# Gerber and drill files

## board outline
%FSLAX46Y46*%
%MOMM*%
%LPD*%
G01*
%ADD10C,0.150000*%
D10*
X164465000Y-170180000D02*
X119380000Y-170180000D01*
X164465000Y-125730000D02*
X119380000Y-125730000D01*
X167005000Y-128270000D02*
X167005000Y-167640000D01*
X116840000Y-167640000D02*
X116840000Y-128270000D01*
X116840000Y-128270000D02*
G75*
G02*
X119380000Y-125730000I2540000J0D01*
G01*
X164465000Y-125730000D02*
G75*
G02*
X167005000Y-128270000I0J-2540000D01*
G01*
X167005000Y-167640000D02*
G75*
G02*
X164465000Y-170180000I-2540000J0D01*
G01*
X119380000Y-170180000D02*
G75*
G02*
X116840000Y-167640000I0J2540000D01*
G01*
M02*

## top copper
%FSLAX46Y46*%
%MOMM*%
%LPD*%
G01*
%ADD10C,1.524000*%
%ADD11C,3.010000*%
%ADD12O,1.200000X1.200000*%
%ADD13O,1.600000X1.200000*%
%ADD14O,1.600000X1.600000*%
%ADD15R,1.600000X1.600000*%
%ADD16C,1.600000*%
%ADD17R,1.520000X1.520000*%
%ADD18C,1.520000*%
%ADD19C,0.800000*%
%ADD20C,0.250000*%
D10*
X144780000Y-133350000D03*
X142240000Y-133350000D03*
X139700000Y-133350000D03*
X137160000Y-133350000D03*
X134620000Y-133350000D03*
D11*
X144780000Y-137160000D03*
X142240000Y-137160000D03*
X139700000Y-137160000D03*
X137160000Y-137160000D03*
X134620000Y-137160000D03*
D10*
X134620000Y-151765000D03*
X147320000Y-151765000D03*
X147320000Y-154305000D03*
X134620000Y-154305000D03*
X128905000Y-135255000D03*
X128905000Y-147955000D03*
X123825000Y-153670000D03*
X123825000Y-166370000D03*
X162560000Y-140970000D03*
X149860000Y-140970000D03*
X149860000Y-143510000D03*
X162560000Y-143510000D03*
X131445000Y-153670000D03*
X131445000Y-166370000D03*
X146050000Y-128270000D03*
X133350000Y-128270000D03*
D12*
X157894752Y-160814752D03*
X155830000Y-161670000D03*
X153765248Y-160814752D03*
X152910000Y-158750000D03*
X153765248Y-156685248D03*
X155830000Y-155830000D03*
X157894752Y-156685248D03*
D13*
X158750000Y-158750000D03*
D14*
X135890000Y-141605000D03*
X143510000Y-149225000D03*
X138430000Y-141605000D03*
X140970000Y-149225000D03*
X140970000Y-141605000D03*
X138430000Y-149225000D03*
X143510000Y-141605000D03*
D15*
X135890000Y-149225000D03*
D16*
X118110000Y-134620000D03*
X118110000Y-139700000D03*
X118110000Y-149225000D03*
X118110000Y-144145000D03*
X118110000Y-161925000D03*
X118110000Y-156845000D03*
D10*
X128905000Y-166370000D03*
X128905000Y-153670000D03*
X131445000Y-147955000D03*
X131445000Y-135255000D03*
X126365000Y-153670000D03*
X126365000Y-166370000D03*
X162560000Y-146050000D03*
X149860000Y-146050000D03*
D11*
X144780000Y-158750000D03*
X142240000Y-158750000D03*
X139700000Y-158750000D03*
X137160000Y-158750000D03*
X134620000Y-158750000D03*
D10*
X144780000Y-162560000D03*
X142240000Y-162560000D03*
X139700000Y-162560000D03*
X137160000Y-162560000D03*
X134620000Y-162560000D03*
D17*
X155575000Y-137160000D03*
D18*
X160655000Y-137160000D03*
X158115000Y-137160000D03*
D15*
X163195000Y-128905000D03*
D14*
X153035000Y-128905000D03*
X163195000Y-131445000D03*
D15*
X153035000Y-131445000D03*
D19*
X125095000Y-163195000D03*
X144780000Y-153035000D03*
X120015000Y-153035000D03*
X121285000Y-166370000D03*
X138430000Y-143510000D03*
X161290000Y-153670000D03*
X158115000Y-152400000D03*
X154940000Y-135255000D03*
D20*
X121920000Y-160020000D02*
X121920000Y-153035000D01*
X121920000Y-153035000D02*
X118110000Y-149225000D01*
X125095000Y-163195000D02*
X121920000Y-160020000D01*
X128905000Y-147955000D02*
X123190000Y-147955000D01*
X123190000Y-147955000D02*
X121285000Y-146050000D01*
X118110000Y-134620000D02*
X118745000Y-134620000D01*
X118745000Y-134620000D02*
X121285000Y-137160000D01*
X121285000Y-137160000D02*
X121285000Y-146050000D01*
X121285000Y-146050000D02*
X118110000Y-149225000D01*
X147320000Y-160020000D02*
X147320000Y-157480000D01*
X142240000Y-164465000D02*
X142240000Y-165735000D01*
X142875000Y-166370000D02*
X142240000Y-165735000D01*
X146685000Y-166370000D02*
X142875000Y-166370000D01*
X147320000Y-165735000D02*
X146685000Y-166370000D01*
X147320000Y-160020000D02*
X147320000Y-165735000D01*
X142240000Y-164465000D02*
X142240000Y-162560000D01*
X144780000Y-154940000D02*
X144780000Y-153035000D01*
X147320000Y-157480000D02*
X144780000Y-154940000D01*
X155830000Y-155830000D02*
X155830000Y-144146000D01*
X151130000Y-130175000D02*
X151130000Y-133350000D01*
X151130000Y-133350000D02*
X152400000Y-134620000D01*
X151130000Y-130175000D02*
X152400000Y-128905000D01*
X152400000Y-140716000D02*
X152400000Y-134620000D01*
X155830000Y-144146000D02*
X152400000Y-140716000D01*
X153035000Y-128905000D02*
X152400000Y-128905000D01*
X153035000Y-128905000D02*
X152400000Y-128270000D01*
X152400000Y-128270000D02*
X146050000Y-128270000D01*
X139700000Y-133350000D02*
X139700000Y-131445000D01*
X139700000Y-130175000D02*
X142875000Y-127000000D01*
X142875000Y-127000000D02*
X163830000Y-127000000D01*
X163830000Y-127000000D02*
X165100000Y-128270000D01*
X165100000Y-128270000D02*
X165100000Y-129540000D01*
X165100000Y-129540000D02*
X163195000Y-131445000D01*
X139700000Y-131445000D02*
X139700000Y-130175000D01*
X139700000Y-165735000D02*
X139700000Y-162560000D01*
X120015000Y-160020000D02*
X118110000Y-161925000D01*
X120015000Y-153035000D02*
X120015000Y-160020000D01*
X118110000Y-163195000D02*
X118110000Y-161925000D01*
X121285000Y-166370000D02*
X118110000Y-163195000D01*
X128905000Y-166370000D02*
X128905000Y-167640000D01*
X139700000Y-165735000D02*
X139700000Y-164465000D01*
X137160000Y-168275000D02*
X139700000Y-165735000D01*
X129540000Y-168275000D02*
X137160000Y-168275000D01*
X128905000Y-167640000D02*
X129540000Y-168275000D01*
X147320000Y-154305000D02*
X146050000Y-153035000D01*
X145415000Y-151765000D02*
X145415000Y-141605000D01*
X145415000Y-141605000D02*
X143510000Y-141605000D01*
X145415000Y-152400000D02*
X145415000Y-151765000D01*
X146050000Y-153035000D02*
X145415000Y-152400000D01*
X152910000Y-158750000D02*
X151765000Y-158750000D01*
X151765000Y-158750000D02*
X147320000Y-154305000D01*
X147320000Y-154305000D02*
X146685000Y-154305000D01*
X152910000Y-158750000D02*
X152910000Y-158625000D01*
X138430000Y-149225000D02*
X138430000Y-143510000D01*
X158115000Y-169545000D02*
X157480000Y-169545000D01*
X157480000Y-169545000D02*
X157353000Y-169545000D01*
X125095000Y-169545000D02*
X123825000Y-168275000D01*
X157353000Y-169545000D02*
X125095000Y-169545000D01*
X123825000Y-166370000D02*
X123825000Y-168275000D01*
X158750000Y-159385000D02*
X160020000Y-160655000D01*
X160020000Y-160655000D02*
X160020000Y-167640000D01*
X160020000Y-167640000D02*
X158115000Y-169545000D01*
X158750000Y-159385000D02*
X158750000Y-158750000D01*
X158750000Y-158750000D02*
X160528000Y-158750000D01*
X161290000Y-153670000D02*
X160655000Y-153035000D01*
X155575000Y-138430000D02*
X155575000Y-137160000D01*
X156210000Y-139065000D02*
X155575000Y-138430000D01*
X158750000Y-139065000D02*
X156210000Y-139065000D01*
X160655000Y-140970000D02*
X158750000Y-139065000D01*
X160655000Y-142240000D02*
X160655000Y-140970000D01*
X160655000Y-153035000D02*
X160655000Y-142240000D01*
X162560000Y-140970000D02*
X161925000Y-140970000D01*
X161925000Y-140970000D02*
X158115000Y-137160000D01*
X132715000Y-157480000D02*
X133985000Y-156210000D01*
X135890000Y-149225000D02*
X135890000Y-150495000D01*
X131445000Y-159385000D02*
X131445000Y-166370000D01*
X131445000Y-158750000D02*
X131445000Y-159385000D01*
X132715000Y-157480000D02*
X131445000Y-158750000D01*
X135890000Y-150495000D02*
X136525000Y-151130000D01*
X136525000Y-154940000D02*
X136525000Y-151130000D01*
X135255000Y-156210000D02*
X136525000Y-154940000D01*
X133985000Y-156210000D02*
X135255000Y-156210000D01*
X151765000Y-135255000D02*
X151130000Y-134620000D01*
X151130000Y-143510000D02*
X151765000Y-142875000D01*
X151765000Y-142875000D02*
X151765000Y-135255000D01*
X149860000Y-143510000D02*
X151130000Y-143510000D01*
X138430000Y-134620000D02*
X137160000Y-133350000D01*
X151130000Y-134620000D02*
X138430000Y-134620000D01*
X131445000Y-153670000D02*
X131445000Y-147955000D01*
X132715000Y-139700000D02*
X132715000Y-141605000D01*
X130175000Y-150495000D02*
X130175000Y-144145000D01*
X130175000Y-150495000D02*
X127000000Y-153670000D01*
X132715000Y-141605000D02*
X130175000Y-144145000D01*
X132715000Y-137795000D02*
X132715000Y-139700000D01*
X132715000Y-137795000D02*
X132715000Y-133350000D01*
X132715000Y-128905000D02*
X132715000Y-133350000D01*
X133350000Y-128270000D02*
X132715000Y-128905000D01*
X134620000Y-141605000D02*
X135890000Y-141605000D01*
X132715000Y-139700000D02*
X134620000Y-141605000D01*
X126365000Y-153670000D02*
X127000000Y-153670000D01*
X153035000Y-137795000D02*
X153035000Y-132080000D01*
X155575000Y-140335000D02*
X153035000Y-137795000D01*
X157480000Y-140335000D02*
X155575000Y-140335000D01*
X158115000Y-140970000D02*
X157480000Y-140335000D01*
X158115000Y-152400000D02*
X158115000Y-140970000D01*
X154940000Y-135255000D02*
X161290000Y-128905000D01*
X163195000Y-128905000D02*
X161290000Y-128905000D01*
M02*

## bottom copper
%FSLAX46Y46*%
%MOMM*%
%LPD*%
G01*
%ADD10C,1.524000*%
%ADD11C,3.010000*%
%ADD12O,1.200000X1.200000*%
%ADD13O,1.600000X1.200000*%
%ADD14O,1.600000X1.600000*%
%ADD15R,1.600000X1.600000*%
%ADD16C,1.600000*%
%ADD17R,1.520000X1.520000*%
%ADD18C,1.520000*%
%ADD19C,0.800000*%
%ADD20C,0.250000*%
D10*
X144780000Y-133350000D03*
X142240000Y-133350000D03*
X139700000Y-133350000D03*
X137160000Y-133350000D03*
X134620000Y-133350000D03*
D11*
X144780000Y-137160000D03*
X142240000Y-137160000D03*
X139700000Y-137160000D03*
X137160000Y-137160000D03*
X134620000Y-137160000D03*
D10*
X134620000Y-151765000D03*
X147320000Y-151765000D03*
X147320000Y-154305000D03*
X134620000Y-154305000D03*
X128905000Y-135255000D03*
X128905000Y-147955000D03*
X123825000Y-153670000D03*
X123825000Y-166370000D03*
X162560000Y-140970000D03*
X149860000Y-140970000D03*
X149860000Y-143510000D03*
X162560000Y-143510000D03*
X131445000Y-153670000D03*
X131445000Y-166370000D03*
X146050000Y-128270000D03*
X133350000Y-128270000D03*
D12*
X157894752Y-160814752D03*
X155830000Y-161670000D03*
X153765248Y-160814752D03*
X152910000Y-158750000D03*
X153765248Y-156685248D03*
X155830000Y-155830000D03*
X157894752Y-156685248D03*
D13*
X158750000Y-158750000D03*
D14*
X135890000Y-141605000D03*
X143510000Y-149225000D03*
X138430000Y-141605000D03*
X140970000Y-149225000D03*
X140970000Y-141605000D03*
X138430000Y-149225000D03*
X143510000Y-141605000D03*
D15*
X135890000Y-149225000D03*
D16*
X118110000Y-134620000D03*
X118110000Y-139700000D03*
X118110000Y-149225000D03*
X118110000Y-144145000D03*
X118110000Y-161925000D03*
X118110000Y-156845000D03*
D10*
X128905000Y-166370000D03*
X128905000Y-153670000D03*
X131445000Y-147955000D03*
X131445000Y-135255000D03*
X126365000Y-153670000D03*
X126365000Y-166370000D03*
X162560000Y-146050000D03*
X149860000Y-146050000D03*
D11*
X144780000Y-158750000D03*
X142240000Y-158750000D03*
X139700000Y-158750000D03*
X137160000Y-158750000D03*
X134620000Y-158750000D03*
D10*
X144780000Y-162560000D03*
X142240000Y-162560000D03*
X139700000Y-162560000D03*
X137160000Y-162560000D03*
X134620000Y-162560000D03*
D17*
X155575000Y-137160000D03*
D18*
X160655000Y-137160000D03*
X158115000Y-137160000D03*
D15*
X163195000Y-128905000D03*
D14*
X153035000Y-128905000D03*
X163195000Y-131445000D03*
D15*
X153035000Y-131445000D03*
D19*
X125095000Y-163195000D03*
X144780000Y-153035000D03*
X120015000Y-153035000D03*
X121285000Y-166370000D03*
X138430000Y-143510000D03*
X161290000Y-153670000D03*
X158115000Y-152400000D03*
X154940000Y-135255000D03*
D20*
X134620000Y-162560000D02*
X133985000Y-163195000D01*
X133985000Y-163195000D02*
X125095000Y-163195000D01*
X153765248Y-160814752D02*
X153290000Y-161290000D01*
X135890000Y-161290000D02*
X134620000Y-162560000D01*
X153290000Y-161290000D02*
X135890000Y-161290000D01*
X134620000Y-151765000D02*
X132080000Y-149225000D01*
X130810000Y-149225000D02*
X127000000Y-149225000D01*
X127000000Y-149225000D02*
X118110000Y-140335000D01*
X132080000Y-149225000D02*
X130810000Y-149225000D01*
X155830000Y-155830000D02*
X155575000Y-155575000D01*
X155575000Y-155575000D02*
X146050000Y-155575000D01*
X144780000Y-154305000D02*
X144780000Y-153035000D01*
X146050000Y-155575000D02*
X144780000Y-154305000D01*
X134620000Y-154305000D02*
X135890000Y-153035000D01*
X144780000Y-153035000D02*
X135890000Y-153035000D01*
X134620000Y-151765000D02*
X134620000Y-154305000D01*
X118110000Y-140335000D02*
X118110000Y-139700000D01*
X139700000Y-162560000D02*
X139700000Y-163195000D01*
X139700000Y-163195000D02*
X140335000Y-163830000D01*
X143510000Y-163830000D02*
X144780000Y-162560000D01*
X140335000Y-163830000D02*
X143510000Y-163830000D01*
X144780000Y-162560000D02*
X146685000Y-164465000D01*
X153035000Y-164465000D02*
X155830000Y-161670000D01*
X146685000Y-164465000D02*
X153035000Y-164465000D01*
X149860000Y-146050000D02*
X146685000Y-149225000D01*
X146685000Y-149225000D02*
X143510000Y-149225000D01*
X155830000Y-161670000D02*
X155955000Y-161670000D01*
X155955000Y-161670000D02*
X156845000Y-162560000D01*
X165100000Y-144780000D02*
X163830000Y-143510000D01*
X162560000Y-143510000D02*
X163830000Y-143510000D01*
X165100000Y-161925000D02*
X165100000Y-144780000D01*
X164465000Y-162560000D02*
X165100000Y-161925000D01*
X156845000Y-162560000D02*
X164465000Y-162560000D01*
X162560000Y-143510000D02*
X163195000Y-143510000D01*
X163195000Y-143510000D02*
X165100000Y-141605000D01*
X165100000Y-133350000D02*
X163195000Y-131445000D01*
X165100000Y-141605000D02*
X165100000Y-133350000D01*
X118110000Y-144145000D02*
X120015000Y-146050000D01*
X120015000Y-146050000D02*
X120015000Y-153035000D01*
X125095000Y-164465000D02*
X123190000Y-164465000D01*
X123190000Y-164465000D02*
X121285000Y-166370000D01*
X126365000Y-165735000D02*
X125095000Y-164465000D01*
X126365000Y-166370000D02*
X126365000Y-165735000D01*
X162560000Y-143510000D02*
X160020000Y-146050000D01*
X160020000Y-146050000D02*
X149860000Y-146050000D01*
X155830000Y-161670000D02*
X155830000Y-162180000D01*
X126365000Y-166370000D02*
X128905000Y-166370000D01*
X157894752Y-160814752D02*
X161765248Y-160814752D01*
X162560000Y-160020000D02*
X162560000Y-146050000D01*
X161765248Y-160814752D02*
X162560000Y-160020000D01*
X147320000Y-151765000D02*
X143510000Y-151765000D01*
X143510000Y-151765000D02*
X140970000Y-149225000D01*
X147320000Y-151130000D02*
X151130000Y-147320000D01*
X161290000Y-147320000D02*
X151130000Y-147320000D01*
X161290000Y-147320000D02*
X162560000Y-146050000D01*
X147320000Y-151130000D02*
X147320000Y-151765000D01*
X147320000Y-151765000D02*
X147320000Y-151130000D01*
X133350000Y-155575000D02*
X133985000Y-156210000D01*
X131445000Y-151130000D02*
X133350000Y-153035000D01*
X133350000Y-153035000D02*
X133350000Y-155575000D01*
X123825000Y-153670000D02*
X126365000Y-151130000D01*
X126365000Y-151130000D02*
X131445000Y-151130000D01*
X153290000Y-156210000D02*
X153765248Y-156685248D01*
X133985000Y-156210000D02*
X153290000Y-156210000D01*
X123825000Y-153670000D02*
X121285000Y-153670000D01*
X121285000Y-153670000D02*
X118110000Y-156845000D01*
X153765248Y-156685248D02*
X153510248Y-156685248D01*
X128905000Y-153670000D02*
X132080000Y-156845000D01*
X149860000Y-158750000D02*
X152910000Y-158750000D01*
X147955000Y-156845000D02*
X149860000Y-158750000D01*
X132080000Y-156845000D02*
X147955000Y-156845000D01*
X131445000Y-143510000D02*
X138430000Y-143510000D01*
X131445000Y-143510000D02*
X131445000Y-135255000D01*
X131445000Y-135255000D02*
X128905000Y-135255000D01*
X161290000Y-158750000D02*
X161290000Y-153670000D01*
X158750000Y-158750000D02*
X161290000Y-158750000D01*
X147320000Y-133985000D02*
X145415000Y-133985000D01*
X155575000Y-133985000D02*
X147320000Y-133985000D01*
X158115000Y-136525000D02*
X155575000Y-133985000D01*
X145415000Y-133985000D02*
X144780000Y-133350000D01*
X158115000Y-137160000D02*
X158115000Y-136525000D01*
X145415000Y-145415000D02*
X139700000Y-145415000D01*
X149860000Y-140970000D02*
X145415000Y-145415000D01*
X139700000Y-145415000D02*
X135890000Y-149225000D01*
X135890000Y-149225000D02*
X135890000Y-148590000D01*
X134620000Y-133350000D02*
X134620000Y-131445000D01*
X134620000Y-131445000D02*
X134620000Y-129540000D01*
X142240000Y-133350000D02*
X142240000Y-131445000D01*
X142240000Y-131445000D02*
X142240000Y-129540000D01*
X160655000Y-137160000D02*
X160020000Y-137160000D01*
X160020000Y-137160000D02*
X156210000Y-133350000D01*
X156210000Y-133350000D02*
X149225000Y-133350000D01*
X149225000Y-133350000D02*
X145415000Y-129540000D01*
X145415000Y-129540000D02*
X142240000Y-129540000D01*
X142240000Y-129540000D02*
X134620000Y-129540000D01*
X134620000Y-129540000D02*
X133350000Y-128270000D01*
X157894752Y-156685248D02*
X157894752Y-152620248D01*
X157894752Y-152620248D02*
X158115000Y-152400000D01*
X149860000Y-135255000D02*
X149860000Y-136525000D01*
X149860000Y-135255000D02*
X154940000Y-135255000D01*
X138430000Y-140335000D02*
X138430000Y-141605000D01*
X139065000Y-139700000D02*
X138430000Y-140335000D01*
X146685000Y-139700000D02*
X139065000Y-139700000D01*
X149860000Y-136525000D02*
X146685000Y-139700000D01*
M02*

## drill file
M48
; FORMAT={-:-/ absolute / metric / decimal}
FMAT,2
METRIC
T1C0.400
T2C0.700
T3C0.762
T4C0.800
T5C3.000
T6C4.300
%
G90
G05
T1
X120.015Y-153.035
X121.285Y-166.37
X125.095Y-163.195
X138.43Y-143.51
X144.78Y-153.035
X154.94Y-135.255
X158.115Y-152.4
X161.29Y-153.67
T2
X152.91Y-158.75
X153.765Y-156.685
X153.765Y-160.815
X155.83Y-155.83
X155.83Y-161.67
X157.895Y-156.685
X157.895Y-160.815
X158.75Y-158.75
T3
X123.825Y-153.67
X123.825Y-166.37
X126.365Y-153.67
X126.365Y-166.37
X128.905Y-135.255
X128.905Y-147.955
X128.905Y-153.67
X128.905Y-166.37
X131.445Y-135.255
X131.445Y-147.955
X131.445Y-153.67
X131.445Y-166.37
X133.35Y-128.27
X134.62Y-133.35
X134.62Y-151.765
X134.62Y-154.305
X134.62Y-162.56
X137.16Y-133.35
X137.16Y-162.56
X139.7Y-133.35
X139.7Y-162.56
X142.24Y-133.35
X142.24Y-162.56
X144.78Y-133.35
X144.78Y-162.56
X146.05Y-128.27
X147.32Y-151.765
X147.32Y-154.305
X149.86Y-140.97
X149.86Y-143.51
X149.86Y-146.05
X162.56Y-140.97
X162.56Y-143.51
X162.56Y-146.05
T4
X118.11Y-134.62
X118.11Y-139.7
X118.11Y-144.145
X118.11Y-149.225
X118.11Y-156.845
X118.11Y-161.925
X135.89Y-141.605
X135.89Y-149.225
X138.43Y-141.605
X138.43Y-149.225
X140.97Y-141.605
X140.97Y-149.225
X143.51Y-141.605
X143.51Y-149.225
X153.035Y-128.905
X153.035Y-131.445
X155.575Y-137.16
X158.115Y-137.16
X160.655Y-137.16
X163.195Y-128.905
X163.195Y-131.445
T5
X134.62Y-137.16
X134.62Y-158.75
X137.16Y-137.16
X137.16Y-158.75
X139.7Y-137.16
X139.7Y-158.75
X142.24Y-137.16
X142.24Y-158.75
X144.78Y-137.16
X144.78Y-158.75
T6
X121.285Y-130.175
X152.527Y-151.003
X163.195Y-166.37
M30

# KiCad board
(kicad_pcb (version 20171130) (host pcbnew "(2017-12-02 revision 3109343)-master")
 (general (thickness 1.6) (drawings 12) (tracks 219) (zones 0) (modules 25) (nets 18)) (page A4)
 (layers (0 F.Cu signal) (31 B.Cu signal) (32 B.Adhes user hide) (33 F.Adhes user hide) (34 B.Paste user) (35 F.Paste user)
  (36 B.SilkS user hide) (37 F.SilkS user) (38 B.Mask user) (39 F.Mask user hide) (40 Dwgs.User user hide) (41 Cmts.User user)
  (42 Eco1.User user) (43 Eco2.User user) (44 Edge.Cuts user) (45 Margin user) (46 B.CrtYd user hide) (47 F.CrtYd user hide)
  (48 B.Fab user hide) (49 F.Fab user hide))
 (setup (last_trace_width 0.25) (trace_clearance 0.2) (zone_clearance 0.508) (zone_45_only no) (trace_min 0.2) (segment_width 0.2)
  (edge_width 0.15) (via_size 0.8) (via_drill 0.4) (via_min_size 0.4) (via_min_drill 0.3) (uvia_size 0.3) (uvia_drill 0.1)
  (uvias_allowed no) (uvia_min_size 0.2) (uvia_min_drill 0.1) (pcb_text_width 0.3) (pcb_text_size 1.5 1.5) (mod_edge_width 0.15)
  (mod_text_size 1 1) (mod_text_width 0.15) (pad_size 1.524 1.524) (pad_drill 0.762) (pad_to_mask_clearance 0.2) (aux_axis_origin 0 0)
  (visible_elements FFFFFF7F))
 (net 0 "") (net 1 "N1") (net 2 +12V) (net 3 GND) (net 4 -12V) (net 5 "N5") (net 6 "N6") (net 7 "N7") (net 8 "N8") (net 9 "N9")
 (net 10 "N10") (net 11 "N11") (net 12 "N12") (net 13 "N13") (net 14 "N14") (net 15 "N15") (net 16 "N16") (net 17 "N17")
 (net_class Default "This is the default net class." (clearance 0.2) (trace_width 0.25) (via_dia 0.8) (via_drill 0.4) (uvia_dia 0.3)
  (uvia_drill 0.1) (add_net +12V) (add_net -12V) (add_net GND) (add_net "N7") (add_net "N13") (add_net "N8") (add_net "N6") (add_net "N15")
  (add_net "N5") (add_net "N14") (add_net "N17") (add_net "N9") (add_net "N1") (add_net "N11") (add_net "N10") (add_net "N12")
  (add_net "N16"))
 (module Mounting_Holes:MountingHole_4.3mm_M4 (layer F.Cu) (at 121.285 130.175)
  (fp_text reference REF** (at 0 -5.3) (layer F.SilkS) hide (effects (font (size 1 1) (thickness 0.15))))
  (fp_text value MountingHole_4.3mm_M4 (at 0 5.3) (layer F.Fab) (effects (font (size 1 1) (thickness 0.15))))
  (pad 1 np_thru_hole circle (at 0 0) (size 4.3 4.3) (drill 4.3) (layers *.Cu *.Mask)))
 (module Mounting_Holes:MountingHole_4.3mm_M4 (layer F.Cu) (at 163.195 166.37)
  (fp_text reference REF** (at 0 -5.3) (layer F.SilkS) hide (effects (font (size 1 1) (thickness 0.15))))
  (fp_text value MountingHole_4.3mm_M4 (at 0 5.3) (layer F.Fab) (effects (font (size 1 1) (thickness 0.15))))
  (pad 1 np_thru_hole circle (at 0 0) (size 4.3 4.3) (drill 4.3) (layers *.Cu *.Mask)))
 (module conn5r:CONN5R (layer F.Cu) (at 139.7 134.62)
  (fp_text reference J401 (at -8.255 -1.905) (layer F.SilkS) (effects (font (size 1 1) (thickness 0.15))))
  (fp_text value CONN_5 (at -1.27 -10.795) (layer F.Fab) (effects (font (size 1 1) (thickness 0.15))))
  (pad 5 thru_hole circle (at 5.08 -1.27) (size 1.524 1.524) (drill 0.762) (layers *.Cu *.Mask) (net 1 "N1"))
  (pad 4 thru_hole circle (at 2.54 -1.27) (size 1.524 1.524) (drill 0.762) (layers *.Cu *.Mask) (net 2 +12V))
  (pad 3 thru_hole circle (at 0 -1.27) (size 1.524 1.524) (drill 0.762) (layers *.Cu *.Mask) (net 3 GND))
  (pad 2 thru_hole circle (at -2.54 -1.27) (size 1.524 1.524) (drill 0.762) (layers *.Cu *.Mask) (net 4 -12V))
  (pad 1 thru_hole circle (at -5.08 -1.27) (size 1.524 1.524) (drill 0.762) (layers *.Cu *.Mask) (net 2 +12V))
  (pad 0 thru_hole circle (at 5.08 2.54) (size 3.01 3.01) (drill 3) (layers *.Cu *.Mask))
  (pad 0 thru_hole circle (at 2.54 2.54) (size 3.01 3.01) (drill 3) (layers *.Cu *.Mask))
  (pad 0 thru_hole circle (at 0 2.54) (size 3.01 3.01) (drill 3) (layers *.Cu *.Mask))
  (pad 0 thru_hole circle (at -2.54 2.54) (size 3.01 3.01) (drill 3) (layers *.Cu *.Mask))
  (pad 0 thru_hole circle (at -5.08 2.54) (size 3.01 3.01) (drill 3) (layers *.Cu)))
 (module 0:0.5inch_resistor (layer F.Cu) (at 139.7 151.765)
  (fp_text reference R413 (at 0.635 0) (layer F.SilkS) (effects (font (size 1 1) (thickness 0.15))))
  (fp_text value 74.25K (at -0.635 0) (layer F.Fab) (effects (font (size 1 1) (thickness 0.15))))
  (pad 1 thru_hole circle (at -5.08 0) (size 1.524 1.524) (drill 0.762) (layers *.Cu *.Mask) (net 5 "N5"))
  (pad 2 thru_hole circle (at 7.62 0) (size 1.524 1.524) (drill 0.762) (layers *.Cu *.Mask) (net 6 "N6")))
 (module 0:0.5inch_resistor (layer F.Cu) (at 139.7 154.305)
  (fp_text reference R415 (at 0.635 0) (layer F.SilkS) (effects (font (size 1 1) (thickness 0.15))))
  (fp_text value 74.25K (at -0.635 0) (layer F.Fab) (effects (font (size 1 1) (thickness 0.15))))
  (pad 2 thru_hole circle (at 7.62 0) (size 1.524 1.524) (drill 0.762) (layers *.Cu *.Mask) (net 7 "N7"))
  (pad 1 thru_hole circle (at -5.08 0) (size 1.524 1.524) (drill 0.762) (layers *.Cu *.Mask) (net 5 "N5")))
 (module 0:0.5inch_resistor (layer F.Cu) (at 128.905 140.335 270)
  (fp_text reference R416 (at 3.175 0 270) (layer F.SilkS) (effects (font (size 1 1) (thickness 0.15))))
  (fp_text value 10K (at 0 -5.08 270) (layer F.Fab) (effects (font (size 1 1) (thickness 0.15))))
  (pad 1 thru_hole circle (at -5.08 0 270) (size 1.524 1.524) (drill 0.762) (layers *.Cu *.Mask) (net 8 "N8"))
  (pad 2 thru_hole circle (at 7.62 0 270) (size 1.524 1.524) (drill 0.762) (layers *.Cu *.Mask) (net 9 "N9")))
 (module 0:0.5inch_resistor (layer F.Cu) (at 123.825 158.75 270)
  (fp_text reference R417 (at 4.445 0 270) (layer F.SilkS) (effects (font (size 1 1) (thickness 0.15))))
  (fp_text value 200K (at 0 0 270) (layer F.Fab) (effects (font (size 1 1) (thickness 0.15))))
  (pad 1 thru_hole circle (at -5.08 0 270) (size 1.524 1.524) (drill 0.762) (layers *.Cu *.Mask) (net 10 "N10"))
  (pad 2 thru_hole circle (at 7.62 0 270) (size 1.524 1.524) (drill 0.762) (layers *.Cu *.Mask) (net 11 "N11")))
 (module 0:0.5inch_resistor (layer F.Cu) (at 157.48 140.97 180)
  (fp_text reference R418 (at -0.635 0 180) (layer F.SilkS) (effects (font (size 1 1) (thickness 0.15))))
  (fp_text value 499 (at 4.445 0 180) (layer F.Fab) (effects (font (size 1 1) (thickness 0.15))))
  (pad 1 thru_hole circle (at -5.08 0 180) (size 1.524 1.524) (drill 0.762) (layers *.Cu *.Mask) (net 1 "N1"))
  (pad 2 thru_hole circle (at 7.62 0 180) (size 1.524 1.524) (drill 0.762) (layers *.Cu *.Mask) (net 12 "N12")))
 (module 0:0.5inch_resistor (layer F.Cu) (at 154.94 143.51)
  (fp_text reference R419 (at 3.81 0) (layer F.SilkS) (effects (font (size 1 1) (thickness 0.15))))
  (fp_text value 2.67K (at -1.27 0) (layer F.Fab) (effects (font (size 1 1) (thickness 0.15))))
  (pad 1 thru_hole circle (at -5.08 0) (size 1.524 1.524) (drill 0.762) (layers *.Cu *.Mask) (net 4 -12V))
  (pad 2 thru_hole circle (at 7.62 0) (size 1.524 1.524) (drill 0.762) (layers *.Cu *.Mask) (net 3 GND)))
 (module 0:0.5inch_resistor (layer F.Cu) (at 131.445 161.29 90)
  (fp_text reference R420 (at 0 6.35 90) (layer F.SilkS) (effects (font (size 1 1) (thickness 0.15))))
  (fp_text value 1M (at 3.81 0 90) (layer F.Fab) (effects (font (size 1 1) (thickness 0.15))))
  (pad 2 thru_hole circle (at 7.62 0 90) (size 1.524 1.524) (drill 0.762) (layers *.Cu *.Mask) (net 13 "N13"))
  (pad 1 thru_hole circle (at -5.08 0 90) (size 1.524 1.524) (drill 0.762) (layers *.Cu *.Mask) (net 12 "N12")))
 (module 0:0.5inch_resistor (layer F.Cu) (at 138.43 128.27)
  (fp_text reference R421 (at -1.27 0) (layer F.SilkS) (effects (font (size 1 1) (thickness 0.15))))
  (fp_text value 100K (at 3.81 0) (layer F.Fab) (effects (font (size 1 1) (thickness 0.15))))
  (pad 2 thru_hole circle (at 7.62 0) (size 1.524 1.524) (drill 0.762) (layers *.Cu *.Mask) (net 5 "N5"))
  (pad 1 thru_hole circle (at -5.08 0) (size 1.524 1.524) (drill 0.762) (layers *.Cu *.Mask) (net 2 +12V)))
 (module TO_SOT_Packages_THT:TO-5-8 (layer F.Cu) (at 158.75 158.75 180)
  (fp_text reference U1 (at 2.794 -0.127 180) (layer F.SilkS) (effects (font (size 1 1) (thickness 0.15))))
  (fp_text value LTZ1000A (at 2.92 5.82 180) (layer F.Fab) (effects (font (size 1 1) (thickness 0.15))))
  (pad 8 thru_hole oval (at 0.855248 -2.064752 180) (size 1.2 1.2) (drill 0.7) (layers *.Cu *.Mask) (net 6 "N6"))
  (pad 7 thru_hole oval (at 2.92 -2.92 180) (size 1.2 1.2) (drill 0.7) (layers *.Cu *.Mask) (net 3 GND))
  (pad 6 thru_hole oval (at 4.984752 -2.064752 180) (size 1.2 1.2) (drill 0.7) (layers *.Cu *.Mask) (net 9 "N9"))
  (pad 5 thru_hole oval (at 5.84 0 180) (size 1.2 1.2) (drill 0.7) (layers *.Cu *.Mask) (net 7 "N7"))
  (pad 4 thru_hole oval (at 4.984752 2.064752 180) (size 1.2 1.2) (drill 0.7) (layers *.Cu *.Mask) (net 10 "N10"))
  (pad 3 thru_hole oval (at 2.92 2.92 180) (size 1.2 1.2) (drill 0.7) (layers *.Cu *.Mask) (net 5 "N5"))
  (pad 2 thru_hole oval (at 0.855248 2.064752 180) (size 1.2 1.2) (drill 0.7) (layers *.Cu *.Mask) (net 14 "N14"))
  (pad 1 thru_hole oval (at 0 0 180) (size 1.6 1.2) (drill 0.7) (layers *.Cu *.Mask) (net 11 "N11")))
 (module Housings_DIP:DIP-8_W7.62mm (layer F.Cu) (at 135.89 149.225 90)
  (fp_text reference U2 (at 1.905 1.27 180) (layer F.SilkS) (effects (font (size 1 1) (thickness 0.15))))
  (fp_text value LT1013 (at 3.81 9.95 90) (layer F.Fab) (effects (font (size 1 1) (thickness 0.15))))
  (pad 8 thru_hole oval (at 7.62 0 90) (size 1.6 1.6) (drill 0.8) (layers *.Cu *.Mask) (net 2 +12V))
  (pad 4 thru_hole oval (at 0 7.62 90) (size 1.6 1.6) (drill 0.8) (layers *.Cu *.Mask) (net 3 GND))
  (pad 7 thru_hole oval (at 7.62 2.54 90) (size 1.6 1.6) (drill 0.8) (layers *.Cu *.Mask) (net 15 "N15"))
  (pad 3 thru_hole oval (at 0 5.08 90) (size 1.6 1.6) (drill 0.8) (layers *.Cu *.Mask) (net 6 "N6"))
  (pad 6 thru_hole oval (at 7.62 5.08 90) (size 1.6 1.6) (drill 0.8) (layers *.Cu *.Mask) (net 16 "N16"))
  (pad 2 thru_hole oval (at 0 2.54 90) (size 1.6 1.6) (drill 0.8) (layers *.Cu *.Mask) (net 8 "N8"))
  (pad 5 thru_hole oval (at 7.62 7.62 90) (size 1.6 1.6) (drill 0.8) (layers *.Cu *.Mask) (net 7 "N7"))
  (pad 1 thru_hole rect (at 0 0 90) (size 1.6 1.6) (drill 0.8) (layers *.Cu *.Mask) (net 12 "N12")))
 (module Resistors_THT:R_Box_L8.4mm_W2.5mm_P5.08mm (layer F.Cu) (at 118.11 139.7 90)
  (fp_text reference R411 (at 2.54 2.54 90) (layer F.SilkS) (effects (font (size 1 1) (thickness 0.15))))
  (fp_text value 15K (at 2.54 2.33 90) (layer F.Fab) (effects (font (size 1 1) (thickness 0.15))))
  (pad 2 thru_hole circle (at 5.08 0 90) (size 1.6 1.6) (drill 0.8) (layers *.Cu *.Mask) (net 9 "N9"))
  (pad 1 thru_hole circle (at 0 0 90) (size 1.6 1.6) (drill 0.8) (layers *.Cu *.Mask) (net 5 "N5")))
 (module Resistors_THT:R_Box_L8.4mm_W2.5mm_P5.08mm (layer F.Cu) (at 118.11 149.225 90)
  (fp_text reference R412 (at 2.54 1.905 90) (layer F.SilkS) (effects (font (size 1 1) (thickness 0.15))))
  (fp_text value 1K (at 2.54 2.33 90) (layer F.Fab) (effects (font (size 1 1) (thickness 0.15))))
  (pad 1 thru_hole circle (at 0 0 90) (size 1.6 1.6) (drill 0.8) (layers *.Cu *.Mask) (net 9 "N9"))
  (pad 2 thru_hole circle (at 5.08 0 90) (size 1.6 1.6) (drill 0.8) (layers *.Cu *.Mask) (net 3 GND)))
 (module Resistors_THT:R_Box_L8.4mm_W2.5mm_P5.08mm (layer F.Cu) (at 118.11 156.845 270)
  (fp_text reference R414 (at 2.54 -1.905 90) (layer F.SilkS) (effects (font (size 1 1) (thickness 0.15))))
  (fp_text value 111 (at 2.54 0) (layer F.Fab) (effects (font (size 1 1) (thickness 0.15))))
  (pad 2 thru_hole circle (at 5.08 0 270) (size 1.6 1.6) (drill 0.8) (layers *.Cu *.Mask) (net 3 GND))
  (pad 1 thru_hole circle (at 0 0 270) (size 1.6 1.6) (drill 0.8) (layers *.Cu *.Mask) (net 10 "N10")))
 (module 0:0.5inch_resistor (layer F.Cu) (at 128.905 158.75 270)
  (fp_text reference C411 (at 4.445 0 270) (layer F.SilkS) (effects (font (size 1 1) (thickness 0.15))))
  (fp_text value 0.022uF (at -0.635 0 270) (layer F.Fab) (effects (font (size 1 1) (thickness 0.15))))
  (pad 2 thru_hole circle (at 7.62 0 270) (size 1.524 1.524) (drill 0.762) (layers *.Cu *.Mask) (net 3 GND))
  (pad 1 thru_hole circle (at -5.08 0 270) (size 1.524 1.524) (drill 0.762) (layers *.Cu *.Mask) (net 7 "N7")))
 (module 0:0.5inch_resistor (layer F.Cu) (at 131.445 142.875 90)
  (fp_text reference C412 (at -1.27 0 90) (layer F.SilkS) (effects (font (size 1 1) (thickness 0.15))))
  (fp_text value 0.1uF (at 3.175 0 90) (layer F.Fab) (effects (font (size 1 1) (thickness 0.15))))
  (pad 1 thru_hole circle (at -5.08 0 90) (size 1.524 1.524) (drill 0.762) (layers *.Cu *.Mask) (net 13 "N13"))
  (pad 2 thru_hole circle (at 7.62 0 90) (size 1.524 1.524) (drill 0.762) (layers *.Cu *.Mask) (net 8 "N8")))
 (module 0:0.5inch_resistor (layer F.Cu) (at 126.365 161.29 90)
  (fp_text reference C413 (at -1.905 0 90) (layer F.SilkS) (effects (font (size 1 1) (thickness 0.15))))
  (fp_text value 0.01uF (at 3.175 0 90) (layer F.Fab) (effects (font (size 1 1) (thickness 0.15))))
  (pad 2 thru_hole circle (at 7.62 0 90) (size 1.524 1.524) (drill 0.762) (layers *.Cu *.Mask) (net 2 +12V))
  (pad 1 thru_hole circle (at -5.08 0 90) (size 1.524 1.524) (drill 0.762) (layers *.Cu *.Mask) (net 3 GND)))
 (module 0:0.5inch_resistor (layer F.Cu) (at 157.48 146.05 180)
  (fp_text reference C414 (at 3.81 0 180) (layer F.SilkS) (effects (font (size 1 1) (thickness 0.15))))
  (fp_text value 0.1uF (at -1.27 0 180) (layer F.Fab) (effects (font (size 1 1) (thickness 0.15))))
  (pad 1 thru_hole circle (at -5.08 0 180) (size 1.524 1.524) (drill 0.762) (layers *.Cu *.Mask) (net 6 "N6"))
  (pad 2 thru_hole circle (at 7.62 0 180) (size 1.524 1.524) (drill 0.762) (layers *.Cu *.Mask) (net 3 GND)))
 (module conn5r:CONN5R (layer F.Cu) (at 139.7 161.29 180)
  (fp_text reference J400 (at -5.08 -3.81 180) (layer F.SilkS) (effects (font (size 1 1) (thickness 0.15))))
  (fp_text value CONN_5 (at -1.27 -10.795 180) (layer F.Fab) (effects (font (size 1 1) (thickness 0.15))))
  (pad 0 thru_hole circle (at -5.08 2.54 180) (size 3.01 3.01) (drill 3) (layers *.Cu))
  (pad 0 thru_hole circle (at -2.54 2.54 180) (size 3.01 3.01) (drill 3) (layers *.Cu *.Mask))
  (pad 0 thru_hole circle (at 0 2.54 180) (size 3.01 3.01) (drill 3) (layers *.Cu *.Mask))
  (pad 0 thru_hole circle (at 2.54 2.54 180) (size 3.01 3.01) (drill 3) (layers *.Cu *.Mask))
  (pad 0 thru_hole circle (at 5.08 2.54 180) (size 3.01 3.01) (drill 3) (layers *.Cu *.Mask))
  (pad 1 thru_hole circle (at -5.08 -1.27 180) (size 1.524 1.524) (drill 0.762) (layers *.Cu *.Mask) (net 3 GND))
  (pad 2 thru_hole circle (at -2.54 -1.27 180) (size 1.524 1.524) (drill 0.762) (layers *.Cu *.Mask) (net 5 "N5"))
  (pad 3 thru_hole circle (at 0 -1.27 180) (size 1.524 1.524) (drill 0.762) (layers *.Cu *.Mask) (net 3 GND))
  (pad 4 thru_hole circle (at 2.54 -1.27 180) (size 1.524 1.524) (drill 0.762) (layers *.Cu *.Mask) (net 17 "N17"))
  (pad 5 thru_hole circle (at 5.08 -1.27 180) (size 1.524 1.524) (drill 0.762) (layers *.Cu *.Mask) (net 9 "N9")))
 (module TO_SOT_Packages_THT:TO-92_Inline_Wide (layer F.Cu) (at 155.575 137.16)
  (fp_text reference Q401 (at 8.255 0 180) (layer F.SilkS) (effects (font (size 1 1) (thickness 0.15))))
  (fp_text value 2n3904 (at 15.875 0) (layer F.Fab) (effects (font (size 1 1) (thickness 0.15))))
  (pad 1 thru_hole rect (at 0 0 90) (size 1.52 1.52) (drill 0.8) (layers *.Cu *.Mask) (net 11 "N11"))
  (pad 3 thru_hole circle (at 5.08 0 90) (size 1.52 1.52) (drill 0.8) (layers *.Cu *.Mask) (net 2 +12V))
  (pad 2 thru_hole circle (at 2.54 0 90) (size 1.52 1.52) (drill 0.8) (layers *.Cu *.Mask) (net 1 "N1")))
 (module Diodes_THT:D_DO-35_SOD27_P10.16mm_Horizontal (layer F.Cu) (at 163.195 128.905 180)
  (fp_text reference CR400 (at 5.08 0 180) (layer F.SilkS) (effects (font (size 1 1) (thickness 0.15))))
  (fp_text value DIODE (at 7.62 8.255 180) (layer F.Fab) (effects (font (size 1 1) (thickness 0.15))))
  (pad 1 thru_hole rect (at 0 0 180) (size 1.6 1.6) (drill 0.8) (layers *.Cu *.Mask) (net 15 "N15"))
  (pad 2 thru_hole oval (at 10.16 0 180) (size 1.6 1.6) (drill 0.8) (layers *.Cu *.Mask) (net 5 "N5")))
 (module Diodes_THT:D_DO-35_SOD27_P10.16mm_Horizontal (layer F.Cu) (at 153.035 131.445)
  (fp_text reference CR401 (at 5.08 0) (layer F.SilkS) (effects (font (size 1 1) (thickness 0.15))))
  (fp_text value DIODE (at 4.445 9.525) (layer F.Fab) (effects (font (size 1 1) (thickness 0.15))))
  (pad 2 thru_hole oval (at 10.16 0) (size 1.6 1.6) (drill 0.8) (layers *.Cu *.Mask) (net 3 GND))
  (pad 1 thru_hole rect (at 0 0) (size 1.6 1.6) (drill 0.8) (layers *.Cu *.Mask) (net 14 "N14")))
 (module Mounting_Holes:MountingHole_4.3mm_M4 (layer F.Cu) (at 152.527 151.003)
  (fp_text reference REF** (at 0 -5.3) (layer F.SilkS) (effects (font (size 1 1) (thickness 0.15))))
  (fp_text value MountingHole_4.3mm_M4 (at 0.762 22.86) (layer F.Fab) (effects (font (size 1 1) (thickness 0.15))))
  (pad 1 np_thru_hole circle (at 0 0) (size 4.3 4.3) (drill 4.3) (layers *.Cu *.Mask)))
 (gr_line (start 164.465 170.18) (end 119.38 170.18) (angle 90) (layer Edge.Cuts) (width 0.15))
 (gr_line (start 164.465 125.73) (end 119.38 125.73) (angle 90) (layer Edge.Cuts) (width 0.15))
 (gr_line (start 167.005 128.27) (end 167.005 167.64) (angle 90) (layer Edge.Cuts) (width 0.15))
 (gr_line (start 116.84 167.64) (end 116.84 128.27) (angle 90) (layer Edge.Cuts) (width 0.15))
 (gr_arc (start 119.38 128.27) (end 116.84 128.27) (angle 90) (layer Edge.Cuts) (width 0.15))
 (gr_arc (start 164.465 128.27) (end 164.465 125.73) (angle 90) (layer Edge.Cuts) (width 0.15))
 (gr_arc (start 164.465 167.64) (end 167.005 167.64) (angle 90) (layer Edge.Cuts) (width 0.15))
 (gr_arc (start 119.38 167.64) (end 119.38 170.18) (angle 90) (layer Edge.Cuts) (width 0.15))
 (segment (start 134.62 162.56) (end 133.985 163.195) (width 0.25) (layer B.Cu) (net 9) (status 400000))
 (segment (start 121.92 160.02) (end 121.92 153.035) (width 0.25) (layer F.Cu) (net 9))
 (segment (start 121.92 153.035) (end 118.11 149.225) (width 0.25) (layer F.Cu) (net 9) (status 800000))
 (via (at 125.095 163.195) (size 0.8) (drill 0.4) (layers F.Cu B.Cu) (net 9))
 (segment (start 125.095 163.195) (end 121.92 160.02) (width 0.25) (layer F.Cu) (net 9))
 (segment (start 133.985 163.195) (end 125.095 163.195) (width 0.25) (layer B.Cu) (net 9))
 (segment (start 153.765248 160.814752) (end 153.29 161.29) (width 0.25) (layer B.Cu) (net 9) (status 400000))
 (segment (start 135.89 161.29) (end 134.62 162.56) (width 0.25) (layer B.Cu) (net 9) (status 800000))
 (segment (start 153.29 161.29) (end 135.89 161.29) (width 0.25) (layer B.Cu) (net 9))
 (segment (start 128.905 147.955) (end 123.19 147.955) (width 0.25) (layer F.Cu) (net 9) (status 400000))
 (segment (start 123.19 147.955) (end 121.285 146.05) (width 0.25) (layer F.Cu) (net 9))
 (segment (start 118.11 134.62) (end 118.745 134.62) (width 0.25) (layer F.Cu) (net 9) (status C00000))
 (segment (start 118.745 134.62) (end 121.285 137.16) (width 0.25) (layer F.Cu) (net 9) (status 400000))
 (segment (start 121.285 137.16) (end 121.285 146.05) (width 0.25) (layer F.Cu) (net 9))
 (segment (start 121.285 146.05) (end 118.11 149.225) (width 0.25) (layer F.Cu) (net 9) (status 800000))
 (segment (start 134.62 151.765) (end 132.08 149.225) (width 0.25) (layer B.Cu) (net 5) (status 400000))
 (segment (start 130.81 149.225) (end 127 149.225) (width 0.25) (layer B.Cu) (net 5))
 (segment (start 127 149.225) (end 118.11 140.335) (width 0.25) (layer B.Cu) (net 5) (status 800000))
 (segment (start 132.08 149.225) (end 130.81 149.225) (width 0.25) (layer B.Cu) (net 5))
 (segment (start 155.83 155.83) (end 155.575 155.575) (width 0.25) (layer B.Cu) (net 5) (status C00000))
 (segment (start 155.575 155.575) (end 146.05 155.575) (width 0.25) (layer B.Cu) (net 5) (status 400000))
 (segment (start 144.78 154.305) (end 144.78 153.035) (width 0.25) (layer B.Cu) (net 5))
 (segment (start 146.05 155.575) (end 144.78 154.305) (width 0.25) (layer B.Cu) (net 5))
 (segment (start 147.32 160.02) (end 147.32 157.48) (width 0.25) (layer F.Cu) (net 5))
 (via (at 144.78 153.035) (size 0.8) (drill 0.4) (layers F.Cu B.Cu) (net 5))
 (segment (start 134.62 154.305) (end 135.89 153.035) (width 0.25) (layer B.Cu) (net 5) (status 400020))
 (segment (start 144.78 153.035) (end 135.89 153.035) (width 0.25) (layer B.Cu) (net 5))
 (segment (start 142.24 164.465) (end 142.24 165.735) (width 0.25) (layer F.Cu) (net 5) (status 400000))
 (segment (start 142.875 166.37) (end 142.24 165.735) (width 0.25) (layer F.Cu) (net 5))
 (segment (start 146.685 166.37) (end 142.875 166.37) (width 0.25) (layer F.Cu) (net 5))
 (segment (start 147.32 165.735) (end 146.685 166.37) (width 0.25) (layer F.Cu) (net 5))
 (segment (start 147.32 160.02) (end 147.32 165.735) (width 0.25) (layer F.Cu) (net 5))
 (segment (start 142.24 164.465) (end 142.24 162.56) (width 0.25) (layer F.Cu) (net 5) (status 800000))
 (segment (start 144.78 154.94) (end 144.78 153.035) (width 0.25) (layer F.Cu) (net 5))
 (segment (start 147.32 157.48) (end 144.78 154.94) (width 0.25) (layer F.Cu) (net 5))
 (segment (start 134.62 151.765) (end 134.62 154.305) (width 0.25) (layer B.Cu) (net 5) (status C00020))
 (segment (start 155.83 155.83) (end 155.83 144.146) (width 0.25) (layer F.Cu) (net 5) (status 400000))
 (segment (start 151.13 130.175) (end 151.13 133.35) (width 0.25) (layer F.Cu) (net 5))
 (segment (start 151.13 133.35) (end 152.4 134.62) (width 0.25) (layer F.Cu) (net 5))
 (segment (start 151.13 130.175) (end 152.4 128.905) (width 0.25) (layer F.Cu) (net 5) (status 800000))
 (segment (start 152.4 140.716) (end 152.4 134.62) (width 0.25) (layer F.Cu) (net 5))
 (segment (start 155.83 144.146) (end 152.4 140.716) (width 0.25) (layer F.Cu) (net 5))
 (segment (start 153.035 128.905) (end 152.4 128.905) (width 0.25) (layer F.Cu) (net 5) (status C00000))
 (segment (start 153.035 128.905) (end 152.4 128.27) (width 0.25) (layer F.Cu) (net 5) (status 400000))
 (segment (start 152.4 128.27) (end 146.05 128.27) (width 0.25) (layer F.Cu) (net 5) (status 800000))
 (segment (start 118.11 140.335) (end 118.11 139.7) (width 0.25) (layer B.Cu) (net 5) (status C00000))
 (segment (start 139.7 133.35) (end 139.7 131.445) (width 0.25) (layer F.Cu) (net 3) (status 400000))
 (segment (start 139.7 130.175) (end 142.875 127) (width 0.25) (layer F.Cu) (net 3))
 (segment (start 142.875 127) (end 163.83 127) (width 0.25) (layer F.Cu) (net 3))
 (segment (start 163.83 127) (end 165.1 128.27) (width 0.25) (layer F.Cu) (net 3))
 (segment (start 165.1 128.27) (end 165.1 129.54) (width 0.25) (layer F.Cu) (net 3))
 (segment (start 165.1 129.54) (end 163.195 131.445) (width 0.25) (layer F.Cu) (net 3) (status 800000))
 (segment (start 139.7 131.445) (end 139.7 130.175) (width 0.25) (layer F.Cu) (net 3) (status 400000))
 (segment (start 139.7 162.56) (end 139.7 163.195) (width 0.25) (layer B.Cu) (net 3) (status C00000))
 (segment (start 139.7 163.195) (end 140.335 163.83) (width 0.25) (layer B.Cu) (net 3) (status 400000))
 (segment (start 143.51 163.83) (end 144.78 162.56) (width 0.25) (layer B.Cu) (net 3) (status 800000))
 (segment (start 140.335 163.83) (end 143.51 163.83) (width 0.25) (layer B.Cu) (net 3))
 (segment (start 139.7 165.735) (end 139.7 162.56) (width 0.25) (layer F.Cu) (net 3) (status 800000))
 (segment (start 144.78 162.56) (end 146.685 164.465) (width 0.25) (layer B.Cu) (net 3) (status 400000))
 (segment (start 153.035 164.465) (end 155.83 161.67) (width 0.25) (layer B.Cu) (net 3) (status 800000))
 (segment (start 146.685 164.465) (end 153.035 164.465) (width 0.25) (layer B.Cu) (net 3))
 (segment (start 149.86 146.05) (end 146.685 149.225) (width 0.25) (layer B.Cu) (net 3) (status 400000))
 (segment (start 146.685 149.225) (end 143.51 149.225) (width 0.25) (layer B.Cu) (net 3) (status 800000))
 (segment (start 155.83 161.67) (end 155.955 161.67) (width 0.25) (layer B.Cu) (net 3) (status C00000))
 (segment (start 155.955 161.67) (end 156.845 162.56) (width 0.25) (layer B.Cu) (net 3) (status 400000))
 (segment (start 165.1 144.78) (end 163.83 143.51) (width 0.25) (layer B.Cu) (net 3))
 (segment (start 162.56 143.51) (end 163.83 143.51) (width 0.25) (layer B.Cu) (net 3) (status 400000))
 (segment (start 165.1 161.925) (end 165.1 144.78) (width 0.25) (layer B.Cu) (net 3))
 (segment (start 164.465 162.56) (end 165.1 161.925) (width 0.25) (layer B.Cu) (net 3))
 (segment (start 156.845 162.56) (end 164.465 162.56) (width 0.25) (layer B.Cu) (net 3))
 (segment (start 162.56 143.51) (end 163.195 143.51) (width 0.25) (layer B.Cu) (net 3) (status C00000))
 (segment (start 163.195 143.51) (end 165.1 141.605) (width 0.25) (layer B.Cu) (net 3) (status 400000))
 (segment (start 165.1 133.35) (end 163.195 131.445) (width 0.25) (layer B.Cu) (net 3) (status 800000))
 (segment (start 165.1 141.605) (end 165.1 133.35) (width 0.25) (layer B.Cu) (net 3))
 (segment (start 118.11 144.145) (end 120.015 146.05) (width 0.25) (layer B.Cu) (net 3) (status 400000))
 (segment (start 120.015 160.02) (end 118.11 161.925) (width 0.25) (layer F.Cu) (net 3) (status 800000))
 (segment (start 120.015 153.035) (end 120.015 160.02) (width 0.25) (layer F.Cu) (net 3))
 (via (at 120.015 153.035) (size 0.8) (drill 0.4) (layers F.Cu B.Cu) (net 3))
 (segment (start 120.015 146.05) (end 120.015 153.035) (width 0.25) (layer B.Cu) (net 3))
 (via (at 121.285 166.37) (size 0.8) (drill 0.4) (layers F.Cu B.Cu) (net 3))
 (segment (start 125.095 164.465) (end 123.19 164.465) (width 0.25) (layer B.Cu) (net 3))
 (segment (start 123.19 164.465) (end 121.285 166.37) (width 0.25) (layer B.Cu) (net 3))
 (segment (start 126.365 165.735) (end 125.095 164.465) (width 0.25) (layer B.Cu) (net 3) (status 400000))
 (segment (start 118.11 163.195) (end 118.11 161.925) (width 0.25) (layer F.Cu) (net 3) (status 800000))
 (segment (start 121.285 166.37) (end 118.11 163.195) (width 0.25) (layer F.Cu) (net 3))
 (segment (start 126.365 166.37) (end 126.365 165.735) (width 0.25) (layer B.Cu) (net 3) (status C00000))
 (segment (start 128.905 166.37) (end 128.905 167.64) (width 0.25) (layer F.Cu) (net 3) (status 400000))
 (segment (start 139.7 165.735) (end 139.7 164.465) (width 0.25) (layer F.Cu) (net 3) (status 800000))
 (segment (start 137.16 168.275) (end 139.7 165.735) (width 0.25) (layer F.Cu) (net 3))
 (segment (start 129.54 168.275) (end 137.16 168.275) (width 0.25) (layer F.Cu) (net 3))
 (segment (start 128.905 167.64) (end 129.54 168.275) (width 0.25) (layer F.Cu) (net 3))
 (segment (start 162.56 143.51) (end 160.02 146.05) (width 0.25) (layer B.Cu) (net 3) (status 400000))
 (segment (start 160.02 146.05) (end 149.86 146.05) (width 0.25) (layer B.Cu) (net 3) (status 800000))
 (segment (start 155.83 161.67) (end 155.83 162.18) (width 0.25) (layer B.Cu) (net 3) (status C00000))
 (segment (start 126.365 166.37) (end 128.905 166.37) (width 0.25) (layer B.Cu) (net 3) (status C00000))
 (segment (start 157.894752 160.814752) (end 161.765248 160.814752) (width 0.25) (layer B.Cu) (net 6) (status 400000))
 (segment (start 162.56 160.02) (end 162.56 146.05) (width 0.25) (layer B.Cu) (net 6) (status 800000))
 (segment (start 161.765248 160.814752) (end 162.56 160.02) (width 0.25) (layer B.Cu) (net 6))
 (segment (start 147.32 151.765) (end 143.51 151.765) (width 0.25) (layer B.Cu) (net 6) (status 400000))
 (segment (start 143.51 151.765) (end 140.97 149.225) (width 0.25) (layer B.Cu) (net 6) (status 800000))
 (segment (start 147.32 151.13) (end 151.13 147.32) (width 0.25) (layer B.Cu) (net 6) (status 400000))
 (segment (start 161.29 147.32) (end 151.13 147.32) (width 0.25) (layer B.Cu) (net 6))
 (segment (start 161.29 147.32) (end 162.56 146.05) (width 0.25) (layer B.Cu) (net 6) (status 800000))
 (segment (start 147.32 151.13) (end 147.32 151.765) (width 0.25) (layer B.Cu) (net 6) (status C00000))
 (segment (start 147.32 151.765) (end 147.32 151.13) (width 0.25) (layer B.Cu) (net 6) (status C00000))
 (segment (start 133.35 155.575) (end 133.985 156.21) (width 0.25) (layer B.Cu) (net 10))
 (segment (start 131.445 151.13) (end 133.35 153.035) (width 0.25) (layer B.Cu) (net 10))
 (segment (start 133.35 153.035) (end 133.35 155.575) (width 0.25) (layer B.Cu) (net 10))
 (segment (start 123.825 153.67) (end 126.365 151.13) (width 0.25) (layer B.Cu) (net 10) (status 400010))
 (segment (start 126.365 151.13) (end 131.445 151.13) (width 0.25) (layer B.Cu) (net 10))
 (segment (start 153.29 156.21) (end 153.765248 156.685248) (width 0.25) (layer B.Cu) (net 10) (status 800000))
 (segment (start 133.985 156.21) (end 153.29 156.21) (width 0.25) (layer B.Cu) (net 10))
 (segment (start 123.825 153.67) (end 121.285 153.67) (width 0.25) (layer B.Cu) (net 10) (status 400010))
 (segment (start 121.285 153.67) (end 118.11 156.845) (width 0.25) (layer B.Cu) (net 10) (status 800000))
 (segment (start 153.765248 156.685248) (end 153.510248 156.685248) (width 0.25) (layer B.Cu) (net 10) (status C00000))
 (segment (start 128.905 153.67) (end 132.08 156.845) (width 0.25) (layer B.Cu) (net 7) (status 400000))
 (segment (start 149.86 158.75) (end 152.91 158.75) (width 0.25) (layer B.Cu) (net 7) (status 800000))
 (segment (start 147.955 156.845) (end 149.86 158.75) (width 0.25) (layer B.Cu) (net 7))
 (segment (start 132.08 156.845) (end 147.955 156.845) (width 0.25) (layer B.Cu) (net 7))
 (segment (start 147.32 154.305) (end 146.05 153.035) (width 0.25) (layer F.Cu) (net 7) (status 400000))
 (segment (start 145.415 151.765) (end 145.415 141.605) (width 0.25) (layer F.Cu) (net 7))
 (segment (start 145.415 141.605) (end 143.51 141.605) (width 0.25) (layer F.Cu) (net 7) (status 800000))
 (segment (start 145.415 152.4) (end 145.415 151.765) (width 0.25) (layer F.Cu) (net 7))
 (segment (start 146.05 153.035) (end 145.415 152.4) (width 0.25) (layer F.Cu) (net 7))
 (segment (start 152.91 158.75) (end 151.765 158.75) (width 0.25) (layer F.Cu) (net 7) (status 400000))
 (segment (start 151.765 158.75) (end 147.32 154.305) (width 0.25) (layer F.Cu) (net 7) (status 800000))
 (segment (start 147.32 154.305) (end 146.685 154.305) (width 0.25) (layer F.Cu) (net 7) (status C00030))
 (segment (start 152.91 158.75) (end 152.91 158.625) (width 0.25) (layer F.Cu) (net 7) (status C00000))
 (segment (start 138.43 149.225) (end 138.43 143.51) (width 0.25) (layer F.Cu) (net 8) (status 400000))
 (via (at 138.43 143.51) (size 0.8) (drill 0.4) (layers F.Cu B.Cu) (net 8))
 (segment (start 131.445 143.51) (end 138.43 143.51) (width 0.25) (layer B.Cu) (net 8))
 (segment (start 131.445 143.51) (end 131.445 135.255) (width 0.25) (layer B.Cu) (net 8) (status 800000))
 (segment (start 131.445 135.255) (end 128.905 135.255) (width 0.25) (layer B.Cu) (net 8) (status C00000))
 (segment (start 158.115 169.545) (end 157.48 169.545) (width 0.25) (layer F.Cu) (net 11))
 (segment (start 157.48 169.545) (end 157.353 169.545) (width 0.25) (layer F.Cu) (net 11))
 (segment (start 125.095 169.545) (end 123.825 168.275) (width 0.25) (layer F.Cu) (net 11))
 (segment (start 157.353 169.545) (end 125.095 169.545) (width 0.25) (layer F.Cu) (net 11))
 (segment (start 123.825 166.37) (end 123.825 168.275) (width 0.25) (layer F.Cu) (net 11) (status 400020))
 (segment (start 158.75 159.385) (end 160.02 160.655) (width 0.25) (layer F.Cu) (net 11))
 (segment (start 160.02 160.655) (end 160.02 167.64) (width 0.25) (layer F.Cu) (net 11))
 (segment (start 160.02 167.64) (end 158.115 169.545) (width 0.25) (layer F.Cu) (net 11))
 (segment (start 158.75 159.385) (end 158.75 158.75) (width 0.25) (layer F.Cu) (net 11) (status 800000))
 (segment (start 158.75 158.75) (end 160.528 158.75) (width 0.25) (layer F.Cu) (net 11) (status 400000))
 (segment (start 161.29 153.67) (end 160.655 153.035) (width 0.25) (layer F.Cu) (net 11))
 (segment (start 161.29 158.75) (end 161.29 153.67) (width 0.25) (layer B.Cu) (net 11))
 (via (at 161.29 153.67) (size 0.8) (drill 0.4) (layers F.Cu B.Cu) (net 11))
 (segment (start 158.75 158.75) (end 161.29 158.75) (width 0.25) (layer B.Cu) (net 11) (status 400000))
 (segment (start 155.575 138.43) (end 155.575 137.16) (width 0.25) (layer F.Cu) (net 11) (status 800000))
 (segment (start 156.21 139.065) (end 155.575 138.43) (width 0.25) (layer F.Cu) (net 11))
 (segment (start 158.75 139.065) (end 156.21 139.065) (width 0.25) (layer F.Cu) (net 11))
 (segment (start 160.655 140.97) (end 158.75 139.065) (width 0.25) (layer F.Cu) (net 11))
 (segment (start 160.655 142.24) (end 160.655 140.97) (width 0.25) (layer F.Cu) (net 11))
 (segment (start 160.655 153.035) (end 160.655 142.24) (width 0.25) (layer F.Cu) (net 11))
 (segment (start 147.32 133.985) (end 145.415 133.985) (width 0.25) (layer B.Cu) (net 1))
 (segment (start 155.575 133.985) (end 147.32 133.985) (width 0.25) (layer B.Cu) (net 1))
 (segment (start 158.115 136.525) (end 155.575 133.985) (width 0.25) (layer B.Cu) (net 1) (status 400000))
 (segment (start 145.415 133.985) (end 144.78 133.35) (width 0.25) (layer B.Cu) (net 1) (status 800000))
 (segment (start 162.56 140.97) (end 161.925 140.97) (width 0.25) (layer F.Cu) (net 1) (status C00000))
 (segment (start 161.925 140.97) (end 158.115 137.16) (width 0.25) (layer F.Cu) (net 1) (status C00000))
 (segment (start 158.115 137.16) (end 158.115 136.525) (width 0.25) (layer B.Cu) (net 1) (status C00000))
 (segment (start 132.715 157.48) (end 133.985 156.21) (width 0.25) (layer F.Cu) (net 12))
 (segment (start 135.89 149.225) (end 135.89 150.495) (width 0.25) (layer F.Cu) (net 12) (status 400010))
 (segment (start 131.445 159.385) (end 131.445 166.37) (width 0.25) (layer F.Cu) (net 12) (status 800000))
 (segment (start 131.445 158.75) (end 131.445 159.385) (width 0.25) (layer F.Cu) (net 12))
 (segment (start 132.715 157.48) (end 131.445 158.75) (width 0.25) (layer F.Cu) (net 12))
 (segment (start 135.89 150.495) (end 136.525 151.13) (width 0.25) (layer F.Cu) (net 12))
 (segment (start 136.525 154.94) (end 136.525 151.13) (width 0.25) (layer F.Cu) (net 12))
 (segment (start 135.255 156.21) (end 136.525 154.94) (width 0.25) (layer F.Cu) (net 12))
 (segment (start 133.985 156.21) (end 135.255 156.21) (width 0.25) (layer F.Cu) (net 12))
 (segment (start 145.415 145.415) (end 139.7 145.415) (width 0.25) (layer B.Cu) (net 12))
 (segment (start 149.86 140.97) (end 145.415 145.415) (width 0.25) (layer B.Cu) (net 12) (status 400000))
 (segment (start 139.7 145.415) (end 135.89 149.225) (width 0.25) (layer B.Cu) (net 12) (status 800000))
 (segment (start 135.89 149.225) (end 135.89 148.59) (width 0.25) (layer B.Cu) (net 12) (status C00030))
 (segment (start 151.765 135.255) (end 151.13 134.62) (width 0.25) (layer F.Cu) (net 4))
 (segment (start 151.13 143.51) (end 151.765 142.875) (width 0.25) (layer F.Cu) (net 4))
 (segment (start 151.765 142.875) (end 151.765 135.255) (width 0.25) (layer F.Cu) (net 4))
 (segment (start 149.86 143.51) (end 151.13 143.51) (width 0.25) (layer F.Cu) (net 4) (status 400000))
 (segment (start 138.43 134.62) (end 137.16 133.35) (width 0.25) (layer F.Cu) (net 4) (status 800000))
 (segment (start 151.13 134.62) (end 138.43 134.62) (width 0.25) (layer F.Cu) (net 4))
 (segment (start 131.445 153.67) (end 131.445 147.955) (width 0.25) (layer F.Cu) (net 13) (status C00000))
 (segment (start 134.62 133.35) (end 134.62 131.445) (width 0.25) (layer B.Cu) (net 2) (status 400000))
 (segment (start 134.62 131.445) (end 134.62 129.54) (width 0.25) (layer B.Cu) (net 2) (status 400000))
 (segment (start 142.24 133.35) (end 142.24 131.445) (width 0.25) (layer B.Cu) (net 2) (status 400000))
 (segment (start 142.24 131.445) (end 142.24 129.54) (width 0.25) (layer B.Cu) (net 2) (status 400000))
 (segment (start 132.715 139.7) (end 132.715 141.605) (width 0.25) (layer F.Cu) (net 2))
 (segment (start 130.175 150.495) (end 130.175 144.145) (width 0.25) (layer F.Cu) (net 2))
 (segment (start 130.175 150.495) (end 127 153.67) (width 0.25) (layer F.Cu) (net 2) (status 800000))
 (segment (start 132.715 141.605) (end 130.175 144.145) (width 0.25) (layer F.Cu) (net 2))
 (segment (start 132.715 137.795) (end 132.715 139.7) (width 0.25) (layer F.Cu) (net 2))
 (segment (start 132.715 137.795) (end 132.715 133.35) (width 0.25) (layer F.Cu) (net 2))
 (segment (start 132.715 128.905) (end 132.715 133.35) (width 0.25) (layer F.Cu) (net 2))
 (segment (start 133.35 128.27) (end 132.715 128.905) (width 0.25) (layer F.Cu) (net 2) (status 400000))
 (segment (start 134.62 141.605) (end 135.89 141.605) (width 0.25) (layer F.Cu) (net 2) (status 800000))
 (segment (start 132.715 139.7) (end 134.62 141.605) (width 0.25) (layer F.Cu) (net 2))
 (segment (start 160.655 137.16) (end 160.02 137.16) (width 0.25) (layer B.Cu) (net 2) (status C00000))
 (segment (start 160.02 137.16) (end 156.21 133.35) (width 0.25) (layer B.Cu) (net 2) (status 400000))
 (segment (start 156.21 133.35) (end 149.225 133.35) (width 0.25) (layer B.Cu) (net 2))
 (segment (start 149.225 133.35) (end 145.415 129.54) (width 0.25) (layer B.Cu) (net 2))
 (segment (start 145.415 129.54) (end 142.24 129.54) (width 0.25) (layer B.Cu) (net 2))
 (segment (start 142.24 129.54) (end 134.62 129.54) (width 0.25) (layer B.Cu) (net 2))
 (segment (start 134.62 129.54) (end 133.35 128.27) (width 0.25) (layer B.Cu) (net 2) (status 800000))
 (segment (start 126.365 153.67) (end 127 153.67) (width 0.25) (layer F.Cu) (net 2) (status C00000))
 (segment (start 157.894752 156.685248) (end 157.894752 152.620248) (width 0.25) (layer B.Cu) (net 14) (status 400000))
 (segment (start 153.035 137.795) (end 153.035 132.08) (width 0.25) (layer F.Cu) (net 14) (status 800000))
 (segment (start 155.575 140.335) (end 153.035 137.795) (width 0.25) (layer F.Cu) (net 14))
 (segment (start 157.48 140.335) (end 155.575 140.335) (width 0.25) (layer F.Cu) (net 14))
 (segment (start 158.115 140.97) (end 157.48 140.335) (width 0.25) (layer F.Cu) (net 14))
 (segment (start 158.115 152.4) (end 158.115 140.97) (width 0.25) (layer F.Cu) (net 14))
 (via (at 158.115 152.4) (size 0.8) (drill 0.4) (layers F.Cu B.Cu) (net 14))
 (segment (start 157.894752 152.620248) (end 158.115 152.4) (width 0.25) (layer B.Cu) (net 14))
 (segment (start 149.86 135.255) (end 149.86 136.525) (width 0.25) (layer B.Cu) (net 15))
 (segment (start 149.86 135.255) (end 154.94 135.255) (width 0.25) (layer B.Cu) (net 15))
 (via (at 154.94 135.255) (size 0.8) (drill 0.4) (layers F.Cu B.Cu) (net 15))
 (segment (start 154.94 135.255) (end 161.29 128.905) (width 0.25) (layer F.Cu) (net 15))
 (segment (start 163.195 128.905) (end 161.29 128.905) (width 0.25) (layer F.Cu) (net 15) (status 400000))
 (segment (start 138.43 140.335) (end 138.43 141.605) (width 0.25) (layer B.Cu) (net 15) (status 800000))
 (segment (start 139.065 139.7) (end 138.43 140.335) (width 0.25) (layer B.Cu) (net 15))
 (segment (start 146.685 139.7) (end 139.065 139.7) (width 0.25) (layer B.Cu) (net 15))
 (segment (start 149.86 136.525) (end 146.685 139.7) (width 0.25) (layer B.Cu) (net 15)))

